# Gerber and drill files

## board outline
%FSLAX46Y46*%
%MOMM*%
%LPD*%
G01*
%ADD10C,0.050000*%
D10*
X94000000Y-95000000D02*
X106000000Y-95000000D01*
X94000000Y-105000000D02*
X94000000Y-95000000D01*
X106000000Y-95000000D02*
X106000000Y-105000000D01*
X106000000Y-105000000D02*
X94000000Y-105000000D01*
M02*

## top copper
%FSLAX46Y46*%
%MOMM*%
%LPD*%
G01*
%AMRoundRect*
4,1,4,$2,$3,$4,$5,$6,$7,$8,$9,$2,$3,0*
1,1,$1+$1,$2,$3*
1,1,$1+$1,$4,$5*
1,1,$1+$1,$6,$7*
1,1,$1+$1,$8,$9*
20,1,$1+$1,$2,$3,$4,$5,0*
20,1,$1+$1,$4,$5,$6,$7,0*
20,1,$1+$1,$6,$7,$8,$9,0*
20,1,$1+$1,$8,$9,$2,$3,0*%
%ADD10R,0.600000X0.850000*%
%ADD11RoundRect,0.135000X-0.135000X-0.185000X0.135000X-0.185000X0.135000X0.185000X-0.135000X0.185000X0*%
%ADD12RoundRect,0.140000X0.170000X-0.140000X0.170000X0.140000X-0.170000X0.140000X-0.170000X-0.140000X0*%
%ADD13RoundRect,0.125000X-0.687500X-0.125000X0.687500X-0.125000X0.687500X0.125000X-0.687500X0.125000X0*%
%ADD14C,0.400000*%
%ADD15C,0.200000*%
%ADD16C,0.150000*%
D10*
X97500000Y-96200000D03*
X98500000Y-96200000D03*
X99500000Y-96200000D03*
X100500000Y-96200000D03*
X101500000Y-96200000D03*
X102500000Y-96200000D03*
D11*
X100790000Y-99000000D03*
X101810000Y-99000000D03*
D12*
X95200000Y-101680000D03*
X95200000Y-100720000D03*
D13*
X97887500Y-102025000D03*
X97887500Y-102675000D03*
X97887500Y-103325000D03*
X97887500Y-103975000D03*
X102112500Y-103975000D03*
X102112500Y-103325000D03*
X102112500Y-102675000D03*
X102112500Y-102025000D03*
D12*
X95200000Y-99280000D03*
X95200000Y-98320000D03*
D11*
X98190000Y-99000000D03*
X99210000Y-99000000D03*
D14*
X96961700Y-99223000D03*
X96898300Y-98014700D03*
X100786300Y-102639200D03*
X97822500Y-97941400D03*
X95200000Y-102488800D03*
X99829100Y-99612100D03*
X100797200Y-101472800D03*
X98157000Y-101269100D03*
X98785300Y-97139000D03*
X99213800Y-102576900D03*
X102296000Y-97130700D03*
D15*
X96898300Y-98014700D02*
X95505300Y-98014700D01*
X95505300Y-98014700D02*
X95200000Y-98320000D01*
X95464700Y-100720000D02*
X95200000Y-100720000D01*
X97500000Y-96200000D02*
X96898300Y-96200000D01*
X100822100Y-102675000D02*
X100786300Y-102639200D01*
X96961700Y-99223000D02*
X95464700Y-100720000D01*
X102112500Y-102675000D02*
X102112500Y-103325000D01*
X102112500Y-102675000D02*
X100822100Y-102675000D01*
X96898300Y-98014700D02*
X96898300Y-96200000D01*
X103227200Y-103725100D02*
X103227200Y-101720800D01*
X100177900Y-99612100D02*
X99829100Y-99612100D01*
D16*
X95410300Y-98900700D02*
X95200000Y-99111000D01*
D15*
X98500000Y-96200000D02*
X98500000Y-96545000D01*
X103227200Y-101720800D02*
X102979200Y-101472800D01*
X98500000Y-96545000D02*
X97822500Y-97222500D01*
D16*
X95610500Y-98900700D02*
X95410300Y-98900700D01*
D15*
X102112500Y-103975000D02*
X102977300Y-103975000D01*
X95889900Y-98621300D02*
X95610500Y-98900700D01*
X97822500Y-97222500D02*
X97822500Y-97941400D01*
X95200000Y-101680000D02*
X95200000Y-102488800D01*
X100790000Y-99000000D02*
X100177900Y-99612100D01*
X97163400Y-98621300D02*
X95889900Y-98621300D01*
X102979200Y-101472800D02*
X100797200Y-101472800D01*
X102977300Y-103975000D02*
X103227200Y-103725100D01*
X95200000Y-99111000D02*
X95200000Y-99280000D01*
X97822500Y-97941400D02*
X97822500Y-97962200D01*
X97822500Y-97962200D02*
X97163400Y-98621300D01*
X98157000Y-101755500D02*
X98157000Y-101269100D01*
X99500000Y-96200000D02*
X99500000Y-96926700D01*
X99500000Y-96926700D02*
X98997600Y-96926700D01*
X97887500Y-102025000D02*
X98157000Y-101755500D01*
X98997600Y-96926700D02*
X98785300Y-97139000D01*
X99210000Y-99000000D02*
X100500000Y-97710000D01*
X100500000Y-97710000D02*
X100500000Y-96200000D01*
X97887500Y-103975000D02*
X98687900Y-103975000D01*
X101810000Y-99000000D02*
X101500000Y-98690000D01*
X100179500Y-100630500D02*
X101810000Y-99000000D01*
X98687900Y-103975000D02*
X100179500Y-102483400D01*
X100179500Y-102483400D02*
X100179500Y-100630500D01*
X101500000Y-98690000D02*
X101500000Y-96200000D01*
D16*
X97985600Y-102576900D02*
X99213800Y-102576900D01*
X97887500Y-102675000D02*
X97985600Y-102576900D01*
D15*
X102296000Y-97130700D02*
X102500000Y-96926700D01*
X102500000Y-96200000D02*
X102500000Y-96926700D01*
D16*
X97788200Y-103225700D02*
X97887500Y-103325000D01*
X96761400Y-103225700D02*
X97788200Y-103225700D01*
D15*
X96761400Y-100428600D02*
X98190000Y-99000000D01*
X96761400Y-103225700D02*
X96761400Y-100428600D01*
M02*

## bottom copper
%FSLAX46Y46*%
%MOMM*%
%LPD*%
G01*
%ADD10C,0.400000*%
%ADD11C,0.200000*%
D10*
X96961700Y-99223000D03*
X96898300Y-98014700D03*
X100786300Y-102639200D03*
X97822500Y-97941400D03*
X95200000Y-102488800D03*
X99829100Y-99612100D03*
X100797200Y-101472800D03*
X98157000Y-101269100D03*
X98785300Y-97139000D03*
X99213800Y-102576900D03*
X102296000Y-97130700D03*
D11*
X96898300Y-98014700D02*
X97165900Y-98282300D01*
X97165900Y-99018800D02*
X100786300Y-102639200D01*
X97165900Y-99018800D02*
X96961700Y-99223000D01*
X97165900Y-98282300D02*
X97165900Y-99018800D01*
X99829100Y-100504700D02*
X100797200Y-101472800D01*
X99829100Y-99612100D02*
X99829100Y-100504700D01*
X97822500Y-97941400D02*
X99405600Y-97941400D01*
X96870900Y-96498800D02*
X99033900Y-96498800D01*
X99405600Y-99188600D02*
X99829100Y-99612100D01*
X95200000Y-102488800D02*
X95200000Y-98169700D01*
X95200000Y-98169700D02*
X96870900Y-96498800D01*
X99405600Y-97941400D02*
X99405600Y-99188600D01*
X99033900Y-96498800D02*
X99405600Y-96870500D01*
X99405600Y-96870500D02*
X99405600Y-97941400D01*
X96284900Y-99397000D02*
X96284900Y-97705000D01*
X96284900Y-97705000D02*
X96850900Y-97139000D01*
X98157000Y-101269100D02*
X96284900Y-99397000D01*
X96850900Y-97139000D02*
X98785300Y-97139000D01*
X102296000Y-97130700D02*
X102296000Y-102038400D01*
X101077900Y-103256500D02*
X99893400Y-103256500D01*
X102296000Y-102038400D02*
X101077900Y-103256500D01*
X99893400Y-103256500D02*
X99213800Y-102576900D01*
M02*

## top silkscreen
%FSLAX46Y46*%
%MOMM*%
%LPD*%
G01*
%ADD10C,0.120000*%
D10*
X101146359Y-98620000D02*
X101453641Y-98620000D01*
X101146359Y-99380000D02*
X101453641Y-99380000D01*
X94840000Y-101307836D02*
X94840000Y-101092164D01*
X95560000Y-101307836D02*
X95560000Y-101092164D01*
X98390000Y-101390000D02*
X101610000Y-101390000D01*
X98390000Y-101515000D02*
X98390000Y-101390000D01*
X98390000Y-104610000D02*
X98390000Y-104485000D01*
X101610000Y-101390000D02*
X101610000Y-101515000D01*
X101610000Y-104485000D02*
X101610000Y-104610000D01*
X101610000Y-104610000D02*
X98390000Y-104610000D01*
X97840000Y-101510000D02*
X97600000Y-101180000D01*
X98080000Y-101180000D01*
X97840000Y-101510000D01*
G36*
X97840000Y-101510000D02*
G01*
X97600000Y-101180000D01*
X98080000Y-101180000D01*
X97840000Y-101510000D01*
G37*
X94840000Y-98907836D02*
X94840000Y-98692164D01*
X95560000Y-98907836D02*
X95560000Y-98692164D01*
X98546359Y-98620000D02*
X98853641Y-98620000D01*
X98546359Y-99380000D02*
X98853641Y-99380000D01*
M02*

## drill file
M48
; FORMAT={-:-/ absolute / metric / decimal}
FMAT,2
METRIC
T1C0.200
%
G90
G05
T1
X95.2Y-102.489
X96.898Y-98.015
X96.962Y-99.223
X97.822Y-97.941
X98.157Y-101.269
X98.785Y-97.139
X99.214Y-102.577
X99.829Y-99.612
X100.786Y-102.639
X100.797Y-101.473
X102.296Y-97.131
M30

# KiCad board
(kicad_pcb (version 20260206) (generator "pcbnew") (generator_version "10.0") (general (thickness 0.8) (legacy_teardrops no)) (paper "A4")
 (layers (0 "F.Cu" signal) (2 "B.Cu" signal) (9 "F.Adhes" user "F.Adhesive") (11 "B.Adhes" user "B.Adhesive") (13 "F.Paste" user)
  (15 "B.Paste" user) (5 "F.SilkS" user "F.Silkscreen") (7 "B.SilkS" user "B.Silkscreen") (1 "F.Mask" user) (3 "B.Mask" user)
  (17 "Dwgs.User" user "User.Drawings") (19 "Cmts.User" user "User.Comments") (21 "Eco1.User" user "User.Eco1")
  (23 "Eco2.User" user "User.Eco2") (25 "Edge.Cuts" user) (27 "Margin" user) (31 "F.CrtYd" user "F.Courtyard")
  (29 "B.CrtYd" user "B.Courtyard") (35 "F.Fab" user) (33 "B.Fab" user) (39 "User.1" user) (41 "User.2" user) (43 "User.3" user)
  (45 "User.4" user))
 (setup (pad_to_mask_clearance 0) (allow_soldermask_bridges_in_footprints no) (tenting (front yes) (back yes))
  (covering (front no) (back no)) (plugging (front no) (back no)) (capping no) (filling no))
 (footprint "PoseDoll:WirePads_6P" (layer "F.Cu") (at 100 96.2)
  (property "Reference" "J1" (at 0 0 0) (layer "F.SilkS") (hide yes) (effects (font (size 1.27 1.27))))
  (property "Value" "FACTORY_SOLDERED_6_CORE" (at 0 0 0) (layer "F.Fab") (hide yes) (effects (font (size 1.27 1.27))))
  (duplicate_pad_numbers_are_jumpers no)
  (pad "1" smd rect (at -2.5 0) (size 0.6 0.85) (layers "F.Cu" "F.Mask") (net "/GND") (thermal_bridge_angle 45))
  (pad "2" smd rect (at -1.5 0) (size 0.6 0.85) (layers "F.Cu" "F.Mask") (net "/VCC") (thermal_bridge_angle 45))
  (pad "3" smd rect (at -0.5 0) (size 0.6 0.85) (layers "F.Cu" "F.Mask") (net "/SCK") (thermal_bridge_angle 45))
  (pad "4" smd rect (at 0.5 0) (size 0.6 0.85) (layers "F.Cu" "F.Mask") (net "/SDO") (thermal_bridge_angle 45))
  (pad "5" smd rect (at 1.5 0) (size 0.6 0.85) (layers "F.Cu" "F.Mask") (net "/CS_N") (thermal_bridge_angle 45))
  (pad "6" smd rect (at 2.5 0) (size 0.6 0.85) (layers "F.Cu" "F.Mask") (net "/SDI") (thermal_bridge_angle 45)))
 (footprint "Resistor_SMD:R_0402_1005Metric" (layer "F.Cu") (at 101.3 99)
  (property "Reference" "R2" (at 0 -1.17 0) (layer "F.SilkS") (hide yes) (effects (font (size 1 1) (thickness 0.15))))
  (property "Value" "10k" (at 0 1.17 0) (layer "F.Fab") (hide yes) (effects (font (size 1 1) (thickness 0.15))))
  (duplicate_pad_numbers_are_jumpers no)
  (fp_line (start -0.153641 -0.38) (end 0.153641 -0.38) (stroke (width 0.12) (type solid)) (layer "F.SilkS"))
  (fp_line (start -0.153641 0.38) (end 0.153641 0.38) (stroke (width 0.12) (type solid)) (layer "F.SilkS"))
  (pad "1" smd roundrect (at -0.51 0) (size 0.54 0.64) (layers "F.Cu" "F.Mask" "F.Paste") (roundrect_rratio 0.25) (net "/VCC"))
  (pad "2" smd roundrect (at 0.51 0) (size 0.54 0.64) (layers "F.Cu" "F.Mask" "F.Paste") (roundrect_rratio 0.25) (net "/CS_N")))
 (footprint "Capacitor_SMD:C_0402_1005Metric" (layer "F.Cu") (at 95.2 101.2 90)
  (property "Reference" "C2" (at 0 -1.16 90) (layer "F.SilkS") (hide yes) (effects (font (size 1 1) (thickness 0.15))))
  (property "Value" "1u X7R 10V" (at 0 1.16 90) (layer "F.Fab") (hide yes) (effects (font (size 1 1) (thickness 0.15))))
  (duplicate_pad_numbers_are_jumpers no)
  (fp_line (start -0.107836 -0.36) (end 0.107836 -0.36) (stroke (width 0.12) (type solid)) (layer "F.SilkS"))
  (fp_line (start -0.107836 0.36) (end 0.107836 0.36) (stroke (width 0.12) (type solid)) (layer "F.SilkS"))
  (pad "1" smd roundrect (at -0.48 0 90) (size 0.56 0.62) (layers "F.Cu" "F.Mask" "F.Paste") (roundrect_rratio 0.25) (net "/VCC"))
  (pad "2" smd roundrect (at 0.48 0 90) (size 0.56 0.62) (layers "F.Cu" "F.Mask" "F.Paste") (roundrect_rratio 0.25) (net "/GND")))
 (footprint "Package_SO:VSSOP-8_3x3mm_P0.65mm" (layer "F.Cu") (at 100 103)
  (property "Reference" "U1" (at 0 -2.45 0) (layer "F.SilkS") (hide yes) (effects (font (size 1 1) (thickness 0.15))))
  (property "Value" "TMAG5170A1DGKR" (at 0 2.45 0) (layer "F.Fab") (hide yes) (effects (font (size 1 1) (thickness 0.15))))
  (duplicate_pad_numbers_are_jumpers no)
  (fp_line (start -1.61 -1.61) (end 1.61 -1.61) (stroke (width 0.12) (type solid)) (layer "F.SilkS"))
  (fp_line (start -1.61 -1.485) (end -1.61 -1.61) (stroke (width 0.12) (type solid)) (layer "F.SilkS"))
  (fp_line (start -1.61 1.61) (end -1.61 1.485) (stroke (width 0.12) (type solid)) (layer "F.SilkS"))
  (fp_line (start 1.61 -1.61) (end 1.61 -1.485) (stroke (width 0.12) (type solid)) (layer "F.SilkS"))
  (fp_line (start 1.61 1.485) (end 1.61 1.61) (stroke (width 0.12) (type solid)) (layer "F.SilkS"))
  (fp_line (start 1.61 1.61) (end -1.61 1.61) (stroke (width 0.12) (type solid)) (layer "F.SilkS"))
  (fp_poly (pts (xy -2.16 -1.49) (xy -2.4 -1.82) (xy -1.92 -1.82)) (stroke (width 0.12) (type solid)) (fill yes) (layer "F.SilkS"))
  (pad "1" smd roundrect (at -2.1125 -0.975) (size 1.625 0.5) (layers "F.Cu" "F.Mask" "F.Paste") (roundrect_rratio 0.25) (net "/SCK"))
  (pad "2" smd roundrect (at -2.1125 -0.325) (size 1.625 0.5) (layers "F.Cu" "F.Mask" "F.Paste") (roundrect_rratio 0.25) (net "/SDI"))
  (pad "3" smd roundrect (at -2.1125 0.325) (size 1.625 0.5) (layers "F.Cu" "F.Mask" "F.Paste") (roundrect_rratio 0.25) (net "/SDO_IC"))
  (pad "4" smd roundrect (at -2.1125 0.975) (size 1.625 0.5) (layers "F.Cu" "F.Mask" "F.Paste") (roundrect_rratio 0.25) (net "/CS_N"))
  (pad "5" smd roundrect (at 2.1125 0.975) (size 1.625 0.5) (layers "F.Cu" "F.Mask" "F.Paste") (roundrect_rratio 0.25) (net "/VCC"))
  (pad "6" smd roundrect (at 2.1125 0.325) (size 1.625 0.5) (layers "F.Cu" "F.Mask" "F.Paste") (roundrect_rratio 0.25) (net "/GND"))
  (pad "7" smd roundrect (at 2.1125 -0.325) (size 1.625 0.5) (layers "F.Cu" "F.Mask" "F.Paste") (roundrect_rratio 0.25) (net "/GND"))
  (pad "8" smd roundrect (at 2.1125 -0.975) (size 1.625 0.5) (layers "F.Cu" "F.Mask" "F.Paste") (roundrect_rratio 0.25)
   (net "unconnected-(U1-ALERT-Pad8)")))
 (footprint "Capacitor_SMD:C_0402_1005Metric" (layer "F.Cu") (at 95.2 98.8 90)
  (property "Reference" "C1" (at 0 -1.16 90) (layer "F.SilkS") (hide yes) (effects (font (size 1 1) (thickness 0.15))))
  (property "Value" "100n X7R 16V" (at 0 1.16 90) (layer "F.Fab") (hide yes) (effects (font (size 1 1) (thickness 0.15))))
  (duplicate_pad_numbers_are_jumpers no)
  (fp_line (start -0.107836 -0.36) (end 0.107836 -0.36) (stroke (width 0.12) (type solid)) (layer "F.SilkS"))
  (fp_line (start -0.107836 0.36) (end 0.107836 0.36) (stroke (width 0.12) (type solid)) (layer "F.SilkS"))
  (pad "1" smd roundrect (at -0.48 0 90) (size 0.56 0.62) (layers "F.Cu" "F.Mask" "F.Paste") (roundrect_rratio 0.25) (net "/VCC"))
  (pad "2" smd roundrect (at 0.48 0 90) (size 0.56 0.62) (layers "F.Cu" "F.Mask" "F.Paste") (roundrect_rratio 0.25) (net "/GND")))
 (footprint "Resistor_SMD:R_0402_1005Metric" (layer "F.Cu") (at 98.7 99)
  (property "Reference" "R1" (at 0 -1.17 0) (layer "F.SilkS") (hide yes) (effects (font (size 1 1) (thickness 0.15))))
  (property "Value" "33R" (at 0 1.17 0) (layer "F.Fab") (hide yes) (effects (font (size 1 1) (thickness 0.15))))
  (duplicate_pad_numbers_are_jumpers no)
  (fp_line (start -0.153641 -0.38) (end 0.153641 -0.38) (stroke (width 0.12) (type solid)) (layer "F.SilkS"))
  (fp_line (start -0.153641 0.38) (end 0.153641 0.38) (stroke (width 0.12) (type solid)) (layer "F.SilkS"))
  (pad "1" smd roundrect (at -0.51 0) (size 0.54 0.64) (layers "F.Cu" "F.Mask" "F.Paste") (roundrect_rratio 0.25) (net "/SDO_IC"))
  (pad "2" smd roundrect (at 0.51 0) (size 0.54 0.64) (layers "F.Cu" "F.Mask" "F.Paste") (roundrect_rratio 0.25) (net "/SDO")))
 (gr_line (start 94 95) (end 106 95) (stroke (width 0.05) (type default)) (layer "Edge.Cuts"))
 (gr_line (start 94 105) (end 94 95) (stroke (width 0.05) (type default)) (layer "Edge.Cuts"))
 (gr_line (start 106 95) (end 106 105) (stroke (width 0.05) (type default)) (layer "Edge.Cuts"))
 (gr_line (start 106 105) (end 94 105) (stroke (width 0.05) (type default)) (layer "Edge.Cuts"))
 (segment (start 96.8983 98.0147) (end 95.5053 98.0147) (width 0.2) (layer "F.Cu") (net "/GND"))
 (segment (start 95.5053 98.0147) (end 95.2 98.32) (width 0.2) (layer "F.Cu") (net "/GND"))
 (segment (start 95.4647 100.72) (end 95.2 100.72) (width 0.2) (layer "F.Cu") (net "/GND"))
 (segment (start 97.5 96.2) (end 96.8983 96.2) (width 0.2) (layer "F.Cu") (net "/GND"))
 (segment (start 100.8221 102.675) (end 100.7863 102.6392) (width 0.2) (layer "F.Cu") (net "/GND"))
 (segment (start 96.9617 99.223) (end 95.4647 100.72) (width 0.2) (layer "F.Cu") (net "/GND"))
 (segment (start 102.1125 102.675) (end 102.1125 103.325) (width 0.2) (layer "F.Cu") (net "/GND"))
 (segment (start 102.1125 102.675) (end 100.8221 102.675) (width 0.2) (layer "F.Cu") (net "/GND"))
 (segment (start 96.8983 98.0147) (end 96.8983 96.2) (width 0.2) (layer "F.Cu") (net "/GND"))
 (via (at 96.9617 99.223) (size 0.4) (drill 0.2) (layers "F.Cu" "B.Cu") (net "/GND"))
 (via (at 96.8983 98.0147) (size 0.4) (drill 0.2) (layers "F.Cu" "B.Cu") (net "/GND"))
 (via (at 100.7863 102.6392) (size 0.4) (drill 0.2) (layers "F.Cu" "B.Cu") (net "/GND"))
 (segment (start 96.8983 98.0147) (end 97.1659 98.2823) (width 0.2) (layer "B.Cu") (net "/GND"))
 (segment (start 97.1659 99.0188) (end 100.7863 102.6392) (width 0.2) (layer "B.Cu") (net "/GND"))
 (segment (start 97.1659 99.0188) (end 96.9617 99.223) (width 0.2) (layer "B.Cu") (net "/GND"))
 (segment (start 97.1659 98.2823) (end 97.1659 99.0188) (width 0.2) (layer "B.Cu") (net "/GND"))
 (segment (start 103.2272 103.7251) (end 103.2272 101.7208) (width 0.2) (layer "F.Cu") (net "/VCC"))
 (segment (start 100.1779 99.6121) (end 99.8291 99.6121) (width 0.2) (layer "F.Cu") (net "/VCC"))
 (segment (start 95.4103 98.9007) (end 95.2 99.111) (width 0.15) (layer "F.Cu") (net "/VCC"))
 (segment (start 98.5 96.2) (end 98.5 96.545) (width 0.2) (layer "F.Cu") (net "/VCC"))
 (segment (start 103.2272 101.7208) (end 102.9792 101.4728) (width 0.2) (layer "F.Cu") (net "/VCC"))
 (segment (start 98.5 96.545) (end 97.8225 97.2225) (width 0.2) (layer "F.Cu") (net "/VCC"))
 (segment (start 95.6105 98.9007) (end 95.4103 98.9007) (width 0.15) (layer "F.Cu") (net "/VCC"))
 (segment (start 102.1125 103.975) (end 102.9773 103.975) (width 0.2) (layer "F.Cu") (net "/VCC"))
 (segment (start 95.8899 98.6213) (end 95.6105 98.9007) (width 0.2) (layer "F.Cu") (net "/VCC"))
 (segment (start 97.8225 97.2225) (end 97.8225 97.9414) (width 0.2) (layer "F.Cu") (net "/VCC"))
 (segment (start 95.2 101.68) (end 95.2 102.4888) (width 0.2) (layer "F.Cu") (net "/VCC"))
 (segment (start 100.79 99) (end 100.1779 99.6121) (width 0.2) (layer "F.Cu") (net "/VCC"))
 (segment (start 97.1634 98.6213) (end 95.8899 98.6213) (width 0.2) (layer "F.Cu") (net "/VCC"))
 (segment (start 102.9792 101.4728) (end 100.7972 101.4728) (width 0.2) (layer "F.Cu") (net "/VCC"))
 (segment (start 102.9773 103.975) (end 103.2272 103.7251) (width 0.2) (layer "F.Cu") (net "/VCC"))
 (segment (start 95.2 99.111) (end 95.2 99.28) (width 0.2) (layer "F.Cu") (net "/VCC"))
 (segment (start 97.8225 97.9414) (end 97.8225 97.9622) (width 0.2) (layer "F.Cu") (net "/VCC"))
 (segment (start 97.8225 97.9622) (end 97.1634 98.6213) (width 0.2) (layer "F.Cu") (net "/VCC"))
 (via (at 97.8225 97.9414) (size 0.4) (drill 0.2) (layers "F.Cu" "B.Cu") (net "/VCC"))
 (via (at 95.2 102.4888) (size 0.4) (drill 0.2) (layers "F.Cu" "B.Cu") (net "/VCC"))
 (via (at 99.8291 99.6121) (size 0.4) (drill 0.2) (layers "F.Cu" "B.Cu") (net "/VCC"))
 (via (at 100.7972 101.4728) (size 0.4) (drill 0.2) (layers "F.Cu" "B.Cu") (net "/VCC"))
 (segment (start 99.8291 100.5047) (end 100.7972 101.4728) (width 0.2) (layer "B.Cu") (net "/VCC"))
 (segment (start 99.8291 99.6121) (end 99.8291 100.5047) (width 0.2) (layer "B.Cu") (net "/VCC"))
 (segment (start 97.8225 97.9414) (end 99.4056 97.9414) (width 0.2) (layer "B.Cu") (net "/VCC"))
 (segment (start 96.8709 96.4988) (end 99.0339 96.4988) (width 0.2) (layer "B.Cu") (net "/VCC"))
 (segment (start 99.4056 99.1886) (end 99.8291 99.6121) (width 0.2) (layer "B.Cu") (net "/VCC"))
 (segment (start 95.2 102.4888) (end 95.2 98.1697) (width 0.2) (layer "B.Cu") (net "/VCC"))
 (segment (start 95.2 98.1697) (end 96.8709 96.4988) (width 0.2) (layer "B.Cu") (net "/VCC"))
 (segment (start 99.4056 97.9414) (end 99.4056 99.1886) (width 0.2) (layer "B.Cu") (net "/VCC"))
 (segment (start 99.0339 96.4988) (end 99.4056 96.8705) (width 0.2) (layer "B.Cu") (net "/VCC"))
 (segment (start 99.4056 96.8705) (end 99.4056 97.9414) (width 0.2) (layer "B.Cu") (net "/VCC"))
 (segment (start 98.157 101.7555) (end 98.157 101.2691) (width 0.2) (layer "F.Cu") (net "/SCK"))
 (segment (start 99.5 96.2) (end 99.5 96.9267) (width 0.2) (layer "F.Cu") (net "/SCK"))
 (segment (start 99.5 96.9267) (end 98.9976 96.9267) (width 0.2) (layer "F.Cu") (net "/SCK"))
 (segment (start 97.8875 102.025) (end 98.157 101.7555) (width 0.2) (layer "F.Cu") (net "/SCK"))
 (segment (start 98.9976 96.9267) (end 98.7853 97.139) (width 0.2) (layer "F.Cu") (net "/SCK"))
 (via (at 98.157 101.2691) (size 0.4) (drill 0.2) (layers "F.Cu" "B.Cu") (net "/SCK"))
 (via (at 98.7853 97.139) (size 0.4) (drill 0.2) (layers "F.Cu" "B.Cu") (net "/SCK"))
 (segment (start 96.2849 99.397) (end 96.2849 97.705) (width 0.2) (layer "B.Cu") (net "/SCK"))
 (segment (start 96.2849 97.705) (end 96.8509 97.139) (width 0.2) (layer "B.Cu") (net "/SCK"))
 (segment (start 98.157 101.2691) (end 96.2849 99.397) (width 0.2) (layer "B.Cu") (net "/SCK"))
 (segment (start 96.8509 97.139) (end 98.7853 97.139) (width 0.2) (layer "B.Cu") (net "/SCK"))
 (segment (start 99.21 99) (end 100.5 97.71) (width 0.2) (layer "F.Cu") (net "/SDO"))
 (segment (start 100.5 97.71) (end 100.5 96.2) (width 0.2) (layer "F.Cu") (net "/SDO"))
 (segment (start 97.8875 103.975) (end 98.6879 103.975) (width 0.2) (layer "F.Cu") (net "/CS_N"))
 (segment (start 101.81 99) (end 101.5 98.69) (width 0.2) (layer "F.Cu") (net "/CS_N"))
 (segment (start 100.1795 100.6305) (end 101.81 99) (width 0.2) (layer "F.Cu") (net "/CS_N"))
 (segment (start 98.6879 103.975) (end 100.1795 102.4834) (width 0.2) (layer "F.Cu") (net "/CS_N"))
 (segment (start 100.1795 102.4834) (end 100.1795 100.6305) (width 0.2) (layer "F.Cu") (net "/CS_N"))
 (segment (start 101.5 98.69) (end 101.5 96.2) (width 0.2) (layer "F.Cu") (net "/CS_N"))
 (segment (start 97.9856 102.5769) (end 99.2138 102.5769) (width 0.15) (layer "F.Cu") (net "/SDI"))
 (segment (start 97.8875 102.675) (end 97.9856 102.5769) (width 0.15) (layer "F.Cu") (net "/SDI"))
 (segment (start 102.296 97.1307) (end 102.5 96.9267) (width 0.2) (layer "F.Cu") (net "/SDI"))
 (segment (start 102.5 96.2) (end 102.5 96.9267) (width 0.2) (layer "F.Cu") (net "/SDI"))
 (via (at 99.2138 102.5769) (size 0.4) (drill 0.2) (layers "F.Cu" "B.Cu") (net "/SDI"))
 (via (at 102.296 97.1307) (size 0.4) (drill 0.2) (layers "F.Cu" "B.Cu") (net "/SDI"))
 (segment (start 102.296 97.1307) (end 102.296 102.0384) (width 0.2) (layer "B.Cu") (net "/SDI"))
 (segment (start 101.0779 103.2565) (end 99.8934 103.2565) (width 0.2) (layer "B.Cu") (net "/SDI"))
 (segment (start 102.296 102.0384) (end 101.0779 103.2565) (width 0.2) (layer "B.Cu") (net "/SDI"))
 (segment (start 99.8934 103.2565) (end 99.2138 102.5769) (width 0.2) (layer "B.Cu") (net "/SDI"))
 (segment (start 97.7882 103.2257) (end 97.8875 103.325) (width 0.15) (layer "F.Cu") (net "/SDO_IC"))
 (segment (start 96.7614 103.2257) (end 97.7882 103.2257) (width 0.15) (layer "F.Cu") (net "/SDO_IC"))
 (segment (start 96.7614 100.4286) (end 98.19 99) (width 0.2) (layer "F.Cu") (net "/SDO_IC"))
 (segment (start 96.7614 103.2257) (end 96.7614 100.4286) (width 0.2) (layer "F.Cu") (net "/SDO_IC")))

